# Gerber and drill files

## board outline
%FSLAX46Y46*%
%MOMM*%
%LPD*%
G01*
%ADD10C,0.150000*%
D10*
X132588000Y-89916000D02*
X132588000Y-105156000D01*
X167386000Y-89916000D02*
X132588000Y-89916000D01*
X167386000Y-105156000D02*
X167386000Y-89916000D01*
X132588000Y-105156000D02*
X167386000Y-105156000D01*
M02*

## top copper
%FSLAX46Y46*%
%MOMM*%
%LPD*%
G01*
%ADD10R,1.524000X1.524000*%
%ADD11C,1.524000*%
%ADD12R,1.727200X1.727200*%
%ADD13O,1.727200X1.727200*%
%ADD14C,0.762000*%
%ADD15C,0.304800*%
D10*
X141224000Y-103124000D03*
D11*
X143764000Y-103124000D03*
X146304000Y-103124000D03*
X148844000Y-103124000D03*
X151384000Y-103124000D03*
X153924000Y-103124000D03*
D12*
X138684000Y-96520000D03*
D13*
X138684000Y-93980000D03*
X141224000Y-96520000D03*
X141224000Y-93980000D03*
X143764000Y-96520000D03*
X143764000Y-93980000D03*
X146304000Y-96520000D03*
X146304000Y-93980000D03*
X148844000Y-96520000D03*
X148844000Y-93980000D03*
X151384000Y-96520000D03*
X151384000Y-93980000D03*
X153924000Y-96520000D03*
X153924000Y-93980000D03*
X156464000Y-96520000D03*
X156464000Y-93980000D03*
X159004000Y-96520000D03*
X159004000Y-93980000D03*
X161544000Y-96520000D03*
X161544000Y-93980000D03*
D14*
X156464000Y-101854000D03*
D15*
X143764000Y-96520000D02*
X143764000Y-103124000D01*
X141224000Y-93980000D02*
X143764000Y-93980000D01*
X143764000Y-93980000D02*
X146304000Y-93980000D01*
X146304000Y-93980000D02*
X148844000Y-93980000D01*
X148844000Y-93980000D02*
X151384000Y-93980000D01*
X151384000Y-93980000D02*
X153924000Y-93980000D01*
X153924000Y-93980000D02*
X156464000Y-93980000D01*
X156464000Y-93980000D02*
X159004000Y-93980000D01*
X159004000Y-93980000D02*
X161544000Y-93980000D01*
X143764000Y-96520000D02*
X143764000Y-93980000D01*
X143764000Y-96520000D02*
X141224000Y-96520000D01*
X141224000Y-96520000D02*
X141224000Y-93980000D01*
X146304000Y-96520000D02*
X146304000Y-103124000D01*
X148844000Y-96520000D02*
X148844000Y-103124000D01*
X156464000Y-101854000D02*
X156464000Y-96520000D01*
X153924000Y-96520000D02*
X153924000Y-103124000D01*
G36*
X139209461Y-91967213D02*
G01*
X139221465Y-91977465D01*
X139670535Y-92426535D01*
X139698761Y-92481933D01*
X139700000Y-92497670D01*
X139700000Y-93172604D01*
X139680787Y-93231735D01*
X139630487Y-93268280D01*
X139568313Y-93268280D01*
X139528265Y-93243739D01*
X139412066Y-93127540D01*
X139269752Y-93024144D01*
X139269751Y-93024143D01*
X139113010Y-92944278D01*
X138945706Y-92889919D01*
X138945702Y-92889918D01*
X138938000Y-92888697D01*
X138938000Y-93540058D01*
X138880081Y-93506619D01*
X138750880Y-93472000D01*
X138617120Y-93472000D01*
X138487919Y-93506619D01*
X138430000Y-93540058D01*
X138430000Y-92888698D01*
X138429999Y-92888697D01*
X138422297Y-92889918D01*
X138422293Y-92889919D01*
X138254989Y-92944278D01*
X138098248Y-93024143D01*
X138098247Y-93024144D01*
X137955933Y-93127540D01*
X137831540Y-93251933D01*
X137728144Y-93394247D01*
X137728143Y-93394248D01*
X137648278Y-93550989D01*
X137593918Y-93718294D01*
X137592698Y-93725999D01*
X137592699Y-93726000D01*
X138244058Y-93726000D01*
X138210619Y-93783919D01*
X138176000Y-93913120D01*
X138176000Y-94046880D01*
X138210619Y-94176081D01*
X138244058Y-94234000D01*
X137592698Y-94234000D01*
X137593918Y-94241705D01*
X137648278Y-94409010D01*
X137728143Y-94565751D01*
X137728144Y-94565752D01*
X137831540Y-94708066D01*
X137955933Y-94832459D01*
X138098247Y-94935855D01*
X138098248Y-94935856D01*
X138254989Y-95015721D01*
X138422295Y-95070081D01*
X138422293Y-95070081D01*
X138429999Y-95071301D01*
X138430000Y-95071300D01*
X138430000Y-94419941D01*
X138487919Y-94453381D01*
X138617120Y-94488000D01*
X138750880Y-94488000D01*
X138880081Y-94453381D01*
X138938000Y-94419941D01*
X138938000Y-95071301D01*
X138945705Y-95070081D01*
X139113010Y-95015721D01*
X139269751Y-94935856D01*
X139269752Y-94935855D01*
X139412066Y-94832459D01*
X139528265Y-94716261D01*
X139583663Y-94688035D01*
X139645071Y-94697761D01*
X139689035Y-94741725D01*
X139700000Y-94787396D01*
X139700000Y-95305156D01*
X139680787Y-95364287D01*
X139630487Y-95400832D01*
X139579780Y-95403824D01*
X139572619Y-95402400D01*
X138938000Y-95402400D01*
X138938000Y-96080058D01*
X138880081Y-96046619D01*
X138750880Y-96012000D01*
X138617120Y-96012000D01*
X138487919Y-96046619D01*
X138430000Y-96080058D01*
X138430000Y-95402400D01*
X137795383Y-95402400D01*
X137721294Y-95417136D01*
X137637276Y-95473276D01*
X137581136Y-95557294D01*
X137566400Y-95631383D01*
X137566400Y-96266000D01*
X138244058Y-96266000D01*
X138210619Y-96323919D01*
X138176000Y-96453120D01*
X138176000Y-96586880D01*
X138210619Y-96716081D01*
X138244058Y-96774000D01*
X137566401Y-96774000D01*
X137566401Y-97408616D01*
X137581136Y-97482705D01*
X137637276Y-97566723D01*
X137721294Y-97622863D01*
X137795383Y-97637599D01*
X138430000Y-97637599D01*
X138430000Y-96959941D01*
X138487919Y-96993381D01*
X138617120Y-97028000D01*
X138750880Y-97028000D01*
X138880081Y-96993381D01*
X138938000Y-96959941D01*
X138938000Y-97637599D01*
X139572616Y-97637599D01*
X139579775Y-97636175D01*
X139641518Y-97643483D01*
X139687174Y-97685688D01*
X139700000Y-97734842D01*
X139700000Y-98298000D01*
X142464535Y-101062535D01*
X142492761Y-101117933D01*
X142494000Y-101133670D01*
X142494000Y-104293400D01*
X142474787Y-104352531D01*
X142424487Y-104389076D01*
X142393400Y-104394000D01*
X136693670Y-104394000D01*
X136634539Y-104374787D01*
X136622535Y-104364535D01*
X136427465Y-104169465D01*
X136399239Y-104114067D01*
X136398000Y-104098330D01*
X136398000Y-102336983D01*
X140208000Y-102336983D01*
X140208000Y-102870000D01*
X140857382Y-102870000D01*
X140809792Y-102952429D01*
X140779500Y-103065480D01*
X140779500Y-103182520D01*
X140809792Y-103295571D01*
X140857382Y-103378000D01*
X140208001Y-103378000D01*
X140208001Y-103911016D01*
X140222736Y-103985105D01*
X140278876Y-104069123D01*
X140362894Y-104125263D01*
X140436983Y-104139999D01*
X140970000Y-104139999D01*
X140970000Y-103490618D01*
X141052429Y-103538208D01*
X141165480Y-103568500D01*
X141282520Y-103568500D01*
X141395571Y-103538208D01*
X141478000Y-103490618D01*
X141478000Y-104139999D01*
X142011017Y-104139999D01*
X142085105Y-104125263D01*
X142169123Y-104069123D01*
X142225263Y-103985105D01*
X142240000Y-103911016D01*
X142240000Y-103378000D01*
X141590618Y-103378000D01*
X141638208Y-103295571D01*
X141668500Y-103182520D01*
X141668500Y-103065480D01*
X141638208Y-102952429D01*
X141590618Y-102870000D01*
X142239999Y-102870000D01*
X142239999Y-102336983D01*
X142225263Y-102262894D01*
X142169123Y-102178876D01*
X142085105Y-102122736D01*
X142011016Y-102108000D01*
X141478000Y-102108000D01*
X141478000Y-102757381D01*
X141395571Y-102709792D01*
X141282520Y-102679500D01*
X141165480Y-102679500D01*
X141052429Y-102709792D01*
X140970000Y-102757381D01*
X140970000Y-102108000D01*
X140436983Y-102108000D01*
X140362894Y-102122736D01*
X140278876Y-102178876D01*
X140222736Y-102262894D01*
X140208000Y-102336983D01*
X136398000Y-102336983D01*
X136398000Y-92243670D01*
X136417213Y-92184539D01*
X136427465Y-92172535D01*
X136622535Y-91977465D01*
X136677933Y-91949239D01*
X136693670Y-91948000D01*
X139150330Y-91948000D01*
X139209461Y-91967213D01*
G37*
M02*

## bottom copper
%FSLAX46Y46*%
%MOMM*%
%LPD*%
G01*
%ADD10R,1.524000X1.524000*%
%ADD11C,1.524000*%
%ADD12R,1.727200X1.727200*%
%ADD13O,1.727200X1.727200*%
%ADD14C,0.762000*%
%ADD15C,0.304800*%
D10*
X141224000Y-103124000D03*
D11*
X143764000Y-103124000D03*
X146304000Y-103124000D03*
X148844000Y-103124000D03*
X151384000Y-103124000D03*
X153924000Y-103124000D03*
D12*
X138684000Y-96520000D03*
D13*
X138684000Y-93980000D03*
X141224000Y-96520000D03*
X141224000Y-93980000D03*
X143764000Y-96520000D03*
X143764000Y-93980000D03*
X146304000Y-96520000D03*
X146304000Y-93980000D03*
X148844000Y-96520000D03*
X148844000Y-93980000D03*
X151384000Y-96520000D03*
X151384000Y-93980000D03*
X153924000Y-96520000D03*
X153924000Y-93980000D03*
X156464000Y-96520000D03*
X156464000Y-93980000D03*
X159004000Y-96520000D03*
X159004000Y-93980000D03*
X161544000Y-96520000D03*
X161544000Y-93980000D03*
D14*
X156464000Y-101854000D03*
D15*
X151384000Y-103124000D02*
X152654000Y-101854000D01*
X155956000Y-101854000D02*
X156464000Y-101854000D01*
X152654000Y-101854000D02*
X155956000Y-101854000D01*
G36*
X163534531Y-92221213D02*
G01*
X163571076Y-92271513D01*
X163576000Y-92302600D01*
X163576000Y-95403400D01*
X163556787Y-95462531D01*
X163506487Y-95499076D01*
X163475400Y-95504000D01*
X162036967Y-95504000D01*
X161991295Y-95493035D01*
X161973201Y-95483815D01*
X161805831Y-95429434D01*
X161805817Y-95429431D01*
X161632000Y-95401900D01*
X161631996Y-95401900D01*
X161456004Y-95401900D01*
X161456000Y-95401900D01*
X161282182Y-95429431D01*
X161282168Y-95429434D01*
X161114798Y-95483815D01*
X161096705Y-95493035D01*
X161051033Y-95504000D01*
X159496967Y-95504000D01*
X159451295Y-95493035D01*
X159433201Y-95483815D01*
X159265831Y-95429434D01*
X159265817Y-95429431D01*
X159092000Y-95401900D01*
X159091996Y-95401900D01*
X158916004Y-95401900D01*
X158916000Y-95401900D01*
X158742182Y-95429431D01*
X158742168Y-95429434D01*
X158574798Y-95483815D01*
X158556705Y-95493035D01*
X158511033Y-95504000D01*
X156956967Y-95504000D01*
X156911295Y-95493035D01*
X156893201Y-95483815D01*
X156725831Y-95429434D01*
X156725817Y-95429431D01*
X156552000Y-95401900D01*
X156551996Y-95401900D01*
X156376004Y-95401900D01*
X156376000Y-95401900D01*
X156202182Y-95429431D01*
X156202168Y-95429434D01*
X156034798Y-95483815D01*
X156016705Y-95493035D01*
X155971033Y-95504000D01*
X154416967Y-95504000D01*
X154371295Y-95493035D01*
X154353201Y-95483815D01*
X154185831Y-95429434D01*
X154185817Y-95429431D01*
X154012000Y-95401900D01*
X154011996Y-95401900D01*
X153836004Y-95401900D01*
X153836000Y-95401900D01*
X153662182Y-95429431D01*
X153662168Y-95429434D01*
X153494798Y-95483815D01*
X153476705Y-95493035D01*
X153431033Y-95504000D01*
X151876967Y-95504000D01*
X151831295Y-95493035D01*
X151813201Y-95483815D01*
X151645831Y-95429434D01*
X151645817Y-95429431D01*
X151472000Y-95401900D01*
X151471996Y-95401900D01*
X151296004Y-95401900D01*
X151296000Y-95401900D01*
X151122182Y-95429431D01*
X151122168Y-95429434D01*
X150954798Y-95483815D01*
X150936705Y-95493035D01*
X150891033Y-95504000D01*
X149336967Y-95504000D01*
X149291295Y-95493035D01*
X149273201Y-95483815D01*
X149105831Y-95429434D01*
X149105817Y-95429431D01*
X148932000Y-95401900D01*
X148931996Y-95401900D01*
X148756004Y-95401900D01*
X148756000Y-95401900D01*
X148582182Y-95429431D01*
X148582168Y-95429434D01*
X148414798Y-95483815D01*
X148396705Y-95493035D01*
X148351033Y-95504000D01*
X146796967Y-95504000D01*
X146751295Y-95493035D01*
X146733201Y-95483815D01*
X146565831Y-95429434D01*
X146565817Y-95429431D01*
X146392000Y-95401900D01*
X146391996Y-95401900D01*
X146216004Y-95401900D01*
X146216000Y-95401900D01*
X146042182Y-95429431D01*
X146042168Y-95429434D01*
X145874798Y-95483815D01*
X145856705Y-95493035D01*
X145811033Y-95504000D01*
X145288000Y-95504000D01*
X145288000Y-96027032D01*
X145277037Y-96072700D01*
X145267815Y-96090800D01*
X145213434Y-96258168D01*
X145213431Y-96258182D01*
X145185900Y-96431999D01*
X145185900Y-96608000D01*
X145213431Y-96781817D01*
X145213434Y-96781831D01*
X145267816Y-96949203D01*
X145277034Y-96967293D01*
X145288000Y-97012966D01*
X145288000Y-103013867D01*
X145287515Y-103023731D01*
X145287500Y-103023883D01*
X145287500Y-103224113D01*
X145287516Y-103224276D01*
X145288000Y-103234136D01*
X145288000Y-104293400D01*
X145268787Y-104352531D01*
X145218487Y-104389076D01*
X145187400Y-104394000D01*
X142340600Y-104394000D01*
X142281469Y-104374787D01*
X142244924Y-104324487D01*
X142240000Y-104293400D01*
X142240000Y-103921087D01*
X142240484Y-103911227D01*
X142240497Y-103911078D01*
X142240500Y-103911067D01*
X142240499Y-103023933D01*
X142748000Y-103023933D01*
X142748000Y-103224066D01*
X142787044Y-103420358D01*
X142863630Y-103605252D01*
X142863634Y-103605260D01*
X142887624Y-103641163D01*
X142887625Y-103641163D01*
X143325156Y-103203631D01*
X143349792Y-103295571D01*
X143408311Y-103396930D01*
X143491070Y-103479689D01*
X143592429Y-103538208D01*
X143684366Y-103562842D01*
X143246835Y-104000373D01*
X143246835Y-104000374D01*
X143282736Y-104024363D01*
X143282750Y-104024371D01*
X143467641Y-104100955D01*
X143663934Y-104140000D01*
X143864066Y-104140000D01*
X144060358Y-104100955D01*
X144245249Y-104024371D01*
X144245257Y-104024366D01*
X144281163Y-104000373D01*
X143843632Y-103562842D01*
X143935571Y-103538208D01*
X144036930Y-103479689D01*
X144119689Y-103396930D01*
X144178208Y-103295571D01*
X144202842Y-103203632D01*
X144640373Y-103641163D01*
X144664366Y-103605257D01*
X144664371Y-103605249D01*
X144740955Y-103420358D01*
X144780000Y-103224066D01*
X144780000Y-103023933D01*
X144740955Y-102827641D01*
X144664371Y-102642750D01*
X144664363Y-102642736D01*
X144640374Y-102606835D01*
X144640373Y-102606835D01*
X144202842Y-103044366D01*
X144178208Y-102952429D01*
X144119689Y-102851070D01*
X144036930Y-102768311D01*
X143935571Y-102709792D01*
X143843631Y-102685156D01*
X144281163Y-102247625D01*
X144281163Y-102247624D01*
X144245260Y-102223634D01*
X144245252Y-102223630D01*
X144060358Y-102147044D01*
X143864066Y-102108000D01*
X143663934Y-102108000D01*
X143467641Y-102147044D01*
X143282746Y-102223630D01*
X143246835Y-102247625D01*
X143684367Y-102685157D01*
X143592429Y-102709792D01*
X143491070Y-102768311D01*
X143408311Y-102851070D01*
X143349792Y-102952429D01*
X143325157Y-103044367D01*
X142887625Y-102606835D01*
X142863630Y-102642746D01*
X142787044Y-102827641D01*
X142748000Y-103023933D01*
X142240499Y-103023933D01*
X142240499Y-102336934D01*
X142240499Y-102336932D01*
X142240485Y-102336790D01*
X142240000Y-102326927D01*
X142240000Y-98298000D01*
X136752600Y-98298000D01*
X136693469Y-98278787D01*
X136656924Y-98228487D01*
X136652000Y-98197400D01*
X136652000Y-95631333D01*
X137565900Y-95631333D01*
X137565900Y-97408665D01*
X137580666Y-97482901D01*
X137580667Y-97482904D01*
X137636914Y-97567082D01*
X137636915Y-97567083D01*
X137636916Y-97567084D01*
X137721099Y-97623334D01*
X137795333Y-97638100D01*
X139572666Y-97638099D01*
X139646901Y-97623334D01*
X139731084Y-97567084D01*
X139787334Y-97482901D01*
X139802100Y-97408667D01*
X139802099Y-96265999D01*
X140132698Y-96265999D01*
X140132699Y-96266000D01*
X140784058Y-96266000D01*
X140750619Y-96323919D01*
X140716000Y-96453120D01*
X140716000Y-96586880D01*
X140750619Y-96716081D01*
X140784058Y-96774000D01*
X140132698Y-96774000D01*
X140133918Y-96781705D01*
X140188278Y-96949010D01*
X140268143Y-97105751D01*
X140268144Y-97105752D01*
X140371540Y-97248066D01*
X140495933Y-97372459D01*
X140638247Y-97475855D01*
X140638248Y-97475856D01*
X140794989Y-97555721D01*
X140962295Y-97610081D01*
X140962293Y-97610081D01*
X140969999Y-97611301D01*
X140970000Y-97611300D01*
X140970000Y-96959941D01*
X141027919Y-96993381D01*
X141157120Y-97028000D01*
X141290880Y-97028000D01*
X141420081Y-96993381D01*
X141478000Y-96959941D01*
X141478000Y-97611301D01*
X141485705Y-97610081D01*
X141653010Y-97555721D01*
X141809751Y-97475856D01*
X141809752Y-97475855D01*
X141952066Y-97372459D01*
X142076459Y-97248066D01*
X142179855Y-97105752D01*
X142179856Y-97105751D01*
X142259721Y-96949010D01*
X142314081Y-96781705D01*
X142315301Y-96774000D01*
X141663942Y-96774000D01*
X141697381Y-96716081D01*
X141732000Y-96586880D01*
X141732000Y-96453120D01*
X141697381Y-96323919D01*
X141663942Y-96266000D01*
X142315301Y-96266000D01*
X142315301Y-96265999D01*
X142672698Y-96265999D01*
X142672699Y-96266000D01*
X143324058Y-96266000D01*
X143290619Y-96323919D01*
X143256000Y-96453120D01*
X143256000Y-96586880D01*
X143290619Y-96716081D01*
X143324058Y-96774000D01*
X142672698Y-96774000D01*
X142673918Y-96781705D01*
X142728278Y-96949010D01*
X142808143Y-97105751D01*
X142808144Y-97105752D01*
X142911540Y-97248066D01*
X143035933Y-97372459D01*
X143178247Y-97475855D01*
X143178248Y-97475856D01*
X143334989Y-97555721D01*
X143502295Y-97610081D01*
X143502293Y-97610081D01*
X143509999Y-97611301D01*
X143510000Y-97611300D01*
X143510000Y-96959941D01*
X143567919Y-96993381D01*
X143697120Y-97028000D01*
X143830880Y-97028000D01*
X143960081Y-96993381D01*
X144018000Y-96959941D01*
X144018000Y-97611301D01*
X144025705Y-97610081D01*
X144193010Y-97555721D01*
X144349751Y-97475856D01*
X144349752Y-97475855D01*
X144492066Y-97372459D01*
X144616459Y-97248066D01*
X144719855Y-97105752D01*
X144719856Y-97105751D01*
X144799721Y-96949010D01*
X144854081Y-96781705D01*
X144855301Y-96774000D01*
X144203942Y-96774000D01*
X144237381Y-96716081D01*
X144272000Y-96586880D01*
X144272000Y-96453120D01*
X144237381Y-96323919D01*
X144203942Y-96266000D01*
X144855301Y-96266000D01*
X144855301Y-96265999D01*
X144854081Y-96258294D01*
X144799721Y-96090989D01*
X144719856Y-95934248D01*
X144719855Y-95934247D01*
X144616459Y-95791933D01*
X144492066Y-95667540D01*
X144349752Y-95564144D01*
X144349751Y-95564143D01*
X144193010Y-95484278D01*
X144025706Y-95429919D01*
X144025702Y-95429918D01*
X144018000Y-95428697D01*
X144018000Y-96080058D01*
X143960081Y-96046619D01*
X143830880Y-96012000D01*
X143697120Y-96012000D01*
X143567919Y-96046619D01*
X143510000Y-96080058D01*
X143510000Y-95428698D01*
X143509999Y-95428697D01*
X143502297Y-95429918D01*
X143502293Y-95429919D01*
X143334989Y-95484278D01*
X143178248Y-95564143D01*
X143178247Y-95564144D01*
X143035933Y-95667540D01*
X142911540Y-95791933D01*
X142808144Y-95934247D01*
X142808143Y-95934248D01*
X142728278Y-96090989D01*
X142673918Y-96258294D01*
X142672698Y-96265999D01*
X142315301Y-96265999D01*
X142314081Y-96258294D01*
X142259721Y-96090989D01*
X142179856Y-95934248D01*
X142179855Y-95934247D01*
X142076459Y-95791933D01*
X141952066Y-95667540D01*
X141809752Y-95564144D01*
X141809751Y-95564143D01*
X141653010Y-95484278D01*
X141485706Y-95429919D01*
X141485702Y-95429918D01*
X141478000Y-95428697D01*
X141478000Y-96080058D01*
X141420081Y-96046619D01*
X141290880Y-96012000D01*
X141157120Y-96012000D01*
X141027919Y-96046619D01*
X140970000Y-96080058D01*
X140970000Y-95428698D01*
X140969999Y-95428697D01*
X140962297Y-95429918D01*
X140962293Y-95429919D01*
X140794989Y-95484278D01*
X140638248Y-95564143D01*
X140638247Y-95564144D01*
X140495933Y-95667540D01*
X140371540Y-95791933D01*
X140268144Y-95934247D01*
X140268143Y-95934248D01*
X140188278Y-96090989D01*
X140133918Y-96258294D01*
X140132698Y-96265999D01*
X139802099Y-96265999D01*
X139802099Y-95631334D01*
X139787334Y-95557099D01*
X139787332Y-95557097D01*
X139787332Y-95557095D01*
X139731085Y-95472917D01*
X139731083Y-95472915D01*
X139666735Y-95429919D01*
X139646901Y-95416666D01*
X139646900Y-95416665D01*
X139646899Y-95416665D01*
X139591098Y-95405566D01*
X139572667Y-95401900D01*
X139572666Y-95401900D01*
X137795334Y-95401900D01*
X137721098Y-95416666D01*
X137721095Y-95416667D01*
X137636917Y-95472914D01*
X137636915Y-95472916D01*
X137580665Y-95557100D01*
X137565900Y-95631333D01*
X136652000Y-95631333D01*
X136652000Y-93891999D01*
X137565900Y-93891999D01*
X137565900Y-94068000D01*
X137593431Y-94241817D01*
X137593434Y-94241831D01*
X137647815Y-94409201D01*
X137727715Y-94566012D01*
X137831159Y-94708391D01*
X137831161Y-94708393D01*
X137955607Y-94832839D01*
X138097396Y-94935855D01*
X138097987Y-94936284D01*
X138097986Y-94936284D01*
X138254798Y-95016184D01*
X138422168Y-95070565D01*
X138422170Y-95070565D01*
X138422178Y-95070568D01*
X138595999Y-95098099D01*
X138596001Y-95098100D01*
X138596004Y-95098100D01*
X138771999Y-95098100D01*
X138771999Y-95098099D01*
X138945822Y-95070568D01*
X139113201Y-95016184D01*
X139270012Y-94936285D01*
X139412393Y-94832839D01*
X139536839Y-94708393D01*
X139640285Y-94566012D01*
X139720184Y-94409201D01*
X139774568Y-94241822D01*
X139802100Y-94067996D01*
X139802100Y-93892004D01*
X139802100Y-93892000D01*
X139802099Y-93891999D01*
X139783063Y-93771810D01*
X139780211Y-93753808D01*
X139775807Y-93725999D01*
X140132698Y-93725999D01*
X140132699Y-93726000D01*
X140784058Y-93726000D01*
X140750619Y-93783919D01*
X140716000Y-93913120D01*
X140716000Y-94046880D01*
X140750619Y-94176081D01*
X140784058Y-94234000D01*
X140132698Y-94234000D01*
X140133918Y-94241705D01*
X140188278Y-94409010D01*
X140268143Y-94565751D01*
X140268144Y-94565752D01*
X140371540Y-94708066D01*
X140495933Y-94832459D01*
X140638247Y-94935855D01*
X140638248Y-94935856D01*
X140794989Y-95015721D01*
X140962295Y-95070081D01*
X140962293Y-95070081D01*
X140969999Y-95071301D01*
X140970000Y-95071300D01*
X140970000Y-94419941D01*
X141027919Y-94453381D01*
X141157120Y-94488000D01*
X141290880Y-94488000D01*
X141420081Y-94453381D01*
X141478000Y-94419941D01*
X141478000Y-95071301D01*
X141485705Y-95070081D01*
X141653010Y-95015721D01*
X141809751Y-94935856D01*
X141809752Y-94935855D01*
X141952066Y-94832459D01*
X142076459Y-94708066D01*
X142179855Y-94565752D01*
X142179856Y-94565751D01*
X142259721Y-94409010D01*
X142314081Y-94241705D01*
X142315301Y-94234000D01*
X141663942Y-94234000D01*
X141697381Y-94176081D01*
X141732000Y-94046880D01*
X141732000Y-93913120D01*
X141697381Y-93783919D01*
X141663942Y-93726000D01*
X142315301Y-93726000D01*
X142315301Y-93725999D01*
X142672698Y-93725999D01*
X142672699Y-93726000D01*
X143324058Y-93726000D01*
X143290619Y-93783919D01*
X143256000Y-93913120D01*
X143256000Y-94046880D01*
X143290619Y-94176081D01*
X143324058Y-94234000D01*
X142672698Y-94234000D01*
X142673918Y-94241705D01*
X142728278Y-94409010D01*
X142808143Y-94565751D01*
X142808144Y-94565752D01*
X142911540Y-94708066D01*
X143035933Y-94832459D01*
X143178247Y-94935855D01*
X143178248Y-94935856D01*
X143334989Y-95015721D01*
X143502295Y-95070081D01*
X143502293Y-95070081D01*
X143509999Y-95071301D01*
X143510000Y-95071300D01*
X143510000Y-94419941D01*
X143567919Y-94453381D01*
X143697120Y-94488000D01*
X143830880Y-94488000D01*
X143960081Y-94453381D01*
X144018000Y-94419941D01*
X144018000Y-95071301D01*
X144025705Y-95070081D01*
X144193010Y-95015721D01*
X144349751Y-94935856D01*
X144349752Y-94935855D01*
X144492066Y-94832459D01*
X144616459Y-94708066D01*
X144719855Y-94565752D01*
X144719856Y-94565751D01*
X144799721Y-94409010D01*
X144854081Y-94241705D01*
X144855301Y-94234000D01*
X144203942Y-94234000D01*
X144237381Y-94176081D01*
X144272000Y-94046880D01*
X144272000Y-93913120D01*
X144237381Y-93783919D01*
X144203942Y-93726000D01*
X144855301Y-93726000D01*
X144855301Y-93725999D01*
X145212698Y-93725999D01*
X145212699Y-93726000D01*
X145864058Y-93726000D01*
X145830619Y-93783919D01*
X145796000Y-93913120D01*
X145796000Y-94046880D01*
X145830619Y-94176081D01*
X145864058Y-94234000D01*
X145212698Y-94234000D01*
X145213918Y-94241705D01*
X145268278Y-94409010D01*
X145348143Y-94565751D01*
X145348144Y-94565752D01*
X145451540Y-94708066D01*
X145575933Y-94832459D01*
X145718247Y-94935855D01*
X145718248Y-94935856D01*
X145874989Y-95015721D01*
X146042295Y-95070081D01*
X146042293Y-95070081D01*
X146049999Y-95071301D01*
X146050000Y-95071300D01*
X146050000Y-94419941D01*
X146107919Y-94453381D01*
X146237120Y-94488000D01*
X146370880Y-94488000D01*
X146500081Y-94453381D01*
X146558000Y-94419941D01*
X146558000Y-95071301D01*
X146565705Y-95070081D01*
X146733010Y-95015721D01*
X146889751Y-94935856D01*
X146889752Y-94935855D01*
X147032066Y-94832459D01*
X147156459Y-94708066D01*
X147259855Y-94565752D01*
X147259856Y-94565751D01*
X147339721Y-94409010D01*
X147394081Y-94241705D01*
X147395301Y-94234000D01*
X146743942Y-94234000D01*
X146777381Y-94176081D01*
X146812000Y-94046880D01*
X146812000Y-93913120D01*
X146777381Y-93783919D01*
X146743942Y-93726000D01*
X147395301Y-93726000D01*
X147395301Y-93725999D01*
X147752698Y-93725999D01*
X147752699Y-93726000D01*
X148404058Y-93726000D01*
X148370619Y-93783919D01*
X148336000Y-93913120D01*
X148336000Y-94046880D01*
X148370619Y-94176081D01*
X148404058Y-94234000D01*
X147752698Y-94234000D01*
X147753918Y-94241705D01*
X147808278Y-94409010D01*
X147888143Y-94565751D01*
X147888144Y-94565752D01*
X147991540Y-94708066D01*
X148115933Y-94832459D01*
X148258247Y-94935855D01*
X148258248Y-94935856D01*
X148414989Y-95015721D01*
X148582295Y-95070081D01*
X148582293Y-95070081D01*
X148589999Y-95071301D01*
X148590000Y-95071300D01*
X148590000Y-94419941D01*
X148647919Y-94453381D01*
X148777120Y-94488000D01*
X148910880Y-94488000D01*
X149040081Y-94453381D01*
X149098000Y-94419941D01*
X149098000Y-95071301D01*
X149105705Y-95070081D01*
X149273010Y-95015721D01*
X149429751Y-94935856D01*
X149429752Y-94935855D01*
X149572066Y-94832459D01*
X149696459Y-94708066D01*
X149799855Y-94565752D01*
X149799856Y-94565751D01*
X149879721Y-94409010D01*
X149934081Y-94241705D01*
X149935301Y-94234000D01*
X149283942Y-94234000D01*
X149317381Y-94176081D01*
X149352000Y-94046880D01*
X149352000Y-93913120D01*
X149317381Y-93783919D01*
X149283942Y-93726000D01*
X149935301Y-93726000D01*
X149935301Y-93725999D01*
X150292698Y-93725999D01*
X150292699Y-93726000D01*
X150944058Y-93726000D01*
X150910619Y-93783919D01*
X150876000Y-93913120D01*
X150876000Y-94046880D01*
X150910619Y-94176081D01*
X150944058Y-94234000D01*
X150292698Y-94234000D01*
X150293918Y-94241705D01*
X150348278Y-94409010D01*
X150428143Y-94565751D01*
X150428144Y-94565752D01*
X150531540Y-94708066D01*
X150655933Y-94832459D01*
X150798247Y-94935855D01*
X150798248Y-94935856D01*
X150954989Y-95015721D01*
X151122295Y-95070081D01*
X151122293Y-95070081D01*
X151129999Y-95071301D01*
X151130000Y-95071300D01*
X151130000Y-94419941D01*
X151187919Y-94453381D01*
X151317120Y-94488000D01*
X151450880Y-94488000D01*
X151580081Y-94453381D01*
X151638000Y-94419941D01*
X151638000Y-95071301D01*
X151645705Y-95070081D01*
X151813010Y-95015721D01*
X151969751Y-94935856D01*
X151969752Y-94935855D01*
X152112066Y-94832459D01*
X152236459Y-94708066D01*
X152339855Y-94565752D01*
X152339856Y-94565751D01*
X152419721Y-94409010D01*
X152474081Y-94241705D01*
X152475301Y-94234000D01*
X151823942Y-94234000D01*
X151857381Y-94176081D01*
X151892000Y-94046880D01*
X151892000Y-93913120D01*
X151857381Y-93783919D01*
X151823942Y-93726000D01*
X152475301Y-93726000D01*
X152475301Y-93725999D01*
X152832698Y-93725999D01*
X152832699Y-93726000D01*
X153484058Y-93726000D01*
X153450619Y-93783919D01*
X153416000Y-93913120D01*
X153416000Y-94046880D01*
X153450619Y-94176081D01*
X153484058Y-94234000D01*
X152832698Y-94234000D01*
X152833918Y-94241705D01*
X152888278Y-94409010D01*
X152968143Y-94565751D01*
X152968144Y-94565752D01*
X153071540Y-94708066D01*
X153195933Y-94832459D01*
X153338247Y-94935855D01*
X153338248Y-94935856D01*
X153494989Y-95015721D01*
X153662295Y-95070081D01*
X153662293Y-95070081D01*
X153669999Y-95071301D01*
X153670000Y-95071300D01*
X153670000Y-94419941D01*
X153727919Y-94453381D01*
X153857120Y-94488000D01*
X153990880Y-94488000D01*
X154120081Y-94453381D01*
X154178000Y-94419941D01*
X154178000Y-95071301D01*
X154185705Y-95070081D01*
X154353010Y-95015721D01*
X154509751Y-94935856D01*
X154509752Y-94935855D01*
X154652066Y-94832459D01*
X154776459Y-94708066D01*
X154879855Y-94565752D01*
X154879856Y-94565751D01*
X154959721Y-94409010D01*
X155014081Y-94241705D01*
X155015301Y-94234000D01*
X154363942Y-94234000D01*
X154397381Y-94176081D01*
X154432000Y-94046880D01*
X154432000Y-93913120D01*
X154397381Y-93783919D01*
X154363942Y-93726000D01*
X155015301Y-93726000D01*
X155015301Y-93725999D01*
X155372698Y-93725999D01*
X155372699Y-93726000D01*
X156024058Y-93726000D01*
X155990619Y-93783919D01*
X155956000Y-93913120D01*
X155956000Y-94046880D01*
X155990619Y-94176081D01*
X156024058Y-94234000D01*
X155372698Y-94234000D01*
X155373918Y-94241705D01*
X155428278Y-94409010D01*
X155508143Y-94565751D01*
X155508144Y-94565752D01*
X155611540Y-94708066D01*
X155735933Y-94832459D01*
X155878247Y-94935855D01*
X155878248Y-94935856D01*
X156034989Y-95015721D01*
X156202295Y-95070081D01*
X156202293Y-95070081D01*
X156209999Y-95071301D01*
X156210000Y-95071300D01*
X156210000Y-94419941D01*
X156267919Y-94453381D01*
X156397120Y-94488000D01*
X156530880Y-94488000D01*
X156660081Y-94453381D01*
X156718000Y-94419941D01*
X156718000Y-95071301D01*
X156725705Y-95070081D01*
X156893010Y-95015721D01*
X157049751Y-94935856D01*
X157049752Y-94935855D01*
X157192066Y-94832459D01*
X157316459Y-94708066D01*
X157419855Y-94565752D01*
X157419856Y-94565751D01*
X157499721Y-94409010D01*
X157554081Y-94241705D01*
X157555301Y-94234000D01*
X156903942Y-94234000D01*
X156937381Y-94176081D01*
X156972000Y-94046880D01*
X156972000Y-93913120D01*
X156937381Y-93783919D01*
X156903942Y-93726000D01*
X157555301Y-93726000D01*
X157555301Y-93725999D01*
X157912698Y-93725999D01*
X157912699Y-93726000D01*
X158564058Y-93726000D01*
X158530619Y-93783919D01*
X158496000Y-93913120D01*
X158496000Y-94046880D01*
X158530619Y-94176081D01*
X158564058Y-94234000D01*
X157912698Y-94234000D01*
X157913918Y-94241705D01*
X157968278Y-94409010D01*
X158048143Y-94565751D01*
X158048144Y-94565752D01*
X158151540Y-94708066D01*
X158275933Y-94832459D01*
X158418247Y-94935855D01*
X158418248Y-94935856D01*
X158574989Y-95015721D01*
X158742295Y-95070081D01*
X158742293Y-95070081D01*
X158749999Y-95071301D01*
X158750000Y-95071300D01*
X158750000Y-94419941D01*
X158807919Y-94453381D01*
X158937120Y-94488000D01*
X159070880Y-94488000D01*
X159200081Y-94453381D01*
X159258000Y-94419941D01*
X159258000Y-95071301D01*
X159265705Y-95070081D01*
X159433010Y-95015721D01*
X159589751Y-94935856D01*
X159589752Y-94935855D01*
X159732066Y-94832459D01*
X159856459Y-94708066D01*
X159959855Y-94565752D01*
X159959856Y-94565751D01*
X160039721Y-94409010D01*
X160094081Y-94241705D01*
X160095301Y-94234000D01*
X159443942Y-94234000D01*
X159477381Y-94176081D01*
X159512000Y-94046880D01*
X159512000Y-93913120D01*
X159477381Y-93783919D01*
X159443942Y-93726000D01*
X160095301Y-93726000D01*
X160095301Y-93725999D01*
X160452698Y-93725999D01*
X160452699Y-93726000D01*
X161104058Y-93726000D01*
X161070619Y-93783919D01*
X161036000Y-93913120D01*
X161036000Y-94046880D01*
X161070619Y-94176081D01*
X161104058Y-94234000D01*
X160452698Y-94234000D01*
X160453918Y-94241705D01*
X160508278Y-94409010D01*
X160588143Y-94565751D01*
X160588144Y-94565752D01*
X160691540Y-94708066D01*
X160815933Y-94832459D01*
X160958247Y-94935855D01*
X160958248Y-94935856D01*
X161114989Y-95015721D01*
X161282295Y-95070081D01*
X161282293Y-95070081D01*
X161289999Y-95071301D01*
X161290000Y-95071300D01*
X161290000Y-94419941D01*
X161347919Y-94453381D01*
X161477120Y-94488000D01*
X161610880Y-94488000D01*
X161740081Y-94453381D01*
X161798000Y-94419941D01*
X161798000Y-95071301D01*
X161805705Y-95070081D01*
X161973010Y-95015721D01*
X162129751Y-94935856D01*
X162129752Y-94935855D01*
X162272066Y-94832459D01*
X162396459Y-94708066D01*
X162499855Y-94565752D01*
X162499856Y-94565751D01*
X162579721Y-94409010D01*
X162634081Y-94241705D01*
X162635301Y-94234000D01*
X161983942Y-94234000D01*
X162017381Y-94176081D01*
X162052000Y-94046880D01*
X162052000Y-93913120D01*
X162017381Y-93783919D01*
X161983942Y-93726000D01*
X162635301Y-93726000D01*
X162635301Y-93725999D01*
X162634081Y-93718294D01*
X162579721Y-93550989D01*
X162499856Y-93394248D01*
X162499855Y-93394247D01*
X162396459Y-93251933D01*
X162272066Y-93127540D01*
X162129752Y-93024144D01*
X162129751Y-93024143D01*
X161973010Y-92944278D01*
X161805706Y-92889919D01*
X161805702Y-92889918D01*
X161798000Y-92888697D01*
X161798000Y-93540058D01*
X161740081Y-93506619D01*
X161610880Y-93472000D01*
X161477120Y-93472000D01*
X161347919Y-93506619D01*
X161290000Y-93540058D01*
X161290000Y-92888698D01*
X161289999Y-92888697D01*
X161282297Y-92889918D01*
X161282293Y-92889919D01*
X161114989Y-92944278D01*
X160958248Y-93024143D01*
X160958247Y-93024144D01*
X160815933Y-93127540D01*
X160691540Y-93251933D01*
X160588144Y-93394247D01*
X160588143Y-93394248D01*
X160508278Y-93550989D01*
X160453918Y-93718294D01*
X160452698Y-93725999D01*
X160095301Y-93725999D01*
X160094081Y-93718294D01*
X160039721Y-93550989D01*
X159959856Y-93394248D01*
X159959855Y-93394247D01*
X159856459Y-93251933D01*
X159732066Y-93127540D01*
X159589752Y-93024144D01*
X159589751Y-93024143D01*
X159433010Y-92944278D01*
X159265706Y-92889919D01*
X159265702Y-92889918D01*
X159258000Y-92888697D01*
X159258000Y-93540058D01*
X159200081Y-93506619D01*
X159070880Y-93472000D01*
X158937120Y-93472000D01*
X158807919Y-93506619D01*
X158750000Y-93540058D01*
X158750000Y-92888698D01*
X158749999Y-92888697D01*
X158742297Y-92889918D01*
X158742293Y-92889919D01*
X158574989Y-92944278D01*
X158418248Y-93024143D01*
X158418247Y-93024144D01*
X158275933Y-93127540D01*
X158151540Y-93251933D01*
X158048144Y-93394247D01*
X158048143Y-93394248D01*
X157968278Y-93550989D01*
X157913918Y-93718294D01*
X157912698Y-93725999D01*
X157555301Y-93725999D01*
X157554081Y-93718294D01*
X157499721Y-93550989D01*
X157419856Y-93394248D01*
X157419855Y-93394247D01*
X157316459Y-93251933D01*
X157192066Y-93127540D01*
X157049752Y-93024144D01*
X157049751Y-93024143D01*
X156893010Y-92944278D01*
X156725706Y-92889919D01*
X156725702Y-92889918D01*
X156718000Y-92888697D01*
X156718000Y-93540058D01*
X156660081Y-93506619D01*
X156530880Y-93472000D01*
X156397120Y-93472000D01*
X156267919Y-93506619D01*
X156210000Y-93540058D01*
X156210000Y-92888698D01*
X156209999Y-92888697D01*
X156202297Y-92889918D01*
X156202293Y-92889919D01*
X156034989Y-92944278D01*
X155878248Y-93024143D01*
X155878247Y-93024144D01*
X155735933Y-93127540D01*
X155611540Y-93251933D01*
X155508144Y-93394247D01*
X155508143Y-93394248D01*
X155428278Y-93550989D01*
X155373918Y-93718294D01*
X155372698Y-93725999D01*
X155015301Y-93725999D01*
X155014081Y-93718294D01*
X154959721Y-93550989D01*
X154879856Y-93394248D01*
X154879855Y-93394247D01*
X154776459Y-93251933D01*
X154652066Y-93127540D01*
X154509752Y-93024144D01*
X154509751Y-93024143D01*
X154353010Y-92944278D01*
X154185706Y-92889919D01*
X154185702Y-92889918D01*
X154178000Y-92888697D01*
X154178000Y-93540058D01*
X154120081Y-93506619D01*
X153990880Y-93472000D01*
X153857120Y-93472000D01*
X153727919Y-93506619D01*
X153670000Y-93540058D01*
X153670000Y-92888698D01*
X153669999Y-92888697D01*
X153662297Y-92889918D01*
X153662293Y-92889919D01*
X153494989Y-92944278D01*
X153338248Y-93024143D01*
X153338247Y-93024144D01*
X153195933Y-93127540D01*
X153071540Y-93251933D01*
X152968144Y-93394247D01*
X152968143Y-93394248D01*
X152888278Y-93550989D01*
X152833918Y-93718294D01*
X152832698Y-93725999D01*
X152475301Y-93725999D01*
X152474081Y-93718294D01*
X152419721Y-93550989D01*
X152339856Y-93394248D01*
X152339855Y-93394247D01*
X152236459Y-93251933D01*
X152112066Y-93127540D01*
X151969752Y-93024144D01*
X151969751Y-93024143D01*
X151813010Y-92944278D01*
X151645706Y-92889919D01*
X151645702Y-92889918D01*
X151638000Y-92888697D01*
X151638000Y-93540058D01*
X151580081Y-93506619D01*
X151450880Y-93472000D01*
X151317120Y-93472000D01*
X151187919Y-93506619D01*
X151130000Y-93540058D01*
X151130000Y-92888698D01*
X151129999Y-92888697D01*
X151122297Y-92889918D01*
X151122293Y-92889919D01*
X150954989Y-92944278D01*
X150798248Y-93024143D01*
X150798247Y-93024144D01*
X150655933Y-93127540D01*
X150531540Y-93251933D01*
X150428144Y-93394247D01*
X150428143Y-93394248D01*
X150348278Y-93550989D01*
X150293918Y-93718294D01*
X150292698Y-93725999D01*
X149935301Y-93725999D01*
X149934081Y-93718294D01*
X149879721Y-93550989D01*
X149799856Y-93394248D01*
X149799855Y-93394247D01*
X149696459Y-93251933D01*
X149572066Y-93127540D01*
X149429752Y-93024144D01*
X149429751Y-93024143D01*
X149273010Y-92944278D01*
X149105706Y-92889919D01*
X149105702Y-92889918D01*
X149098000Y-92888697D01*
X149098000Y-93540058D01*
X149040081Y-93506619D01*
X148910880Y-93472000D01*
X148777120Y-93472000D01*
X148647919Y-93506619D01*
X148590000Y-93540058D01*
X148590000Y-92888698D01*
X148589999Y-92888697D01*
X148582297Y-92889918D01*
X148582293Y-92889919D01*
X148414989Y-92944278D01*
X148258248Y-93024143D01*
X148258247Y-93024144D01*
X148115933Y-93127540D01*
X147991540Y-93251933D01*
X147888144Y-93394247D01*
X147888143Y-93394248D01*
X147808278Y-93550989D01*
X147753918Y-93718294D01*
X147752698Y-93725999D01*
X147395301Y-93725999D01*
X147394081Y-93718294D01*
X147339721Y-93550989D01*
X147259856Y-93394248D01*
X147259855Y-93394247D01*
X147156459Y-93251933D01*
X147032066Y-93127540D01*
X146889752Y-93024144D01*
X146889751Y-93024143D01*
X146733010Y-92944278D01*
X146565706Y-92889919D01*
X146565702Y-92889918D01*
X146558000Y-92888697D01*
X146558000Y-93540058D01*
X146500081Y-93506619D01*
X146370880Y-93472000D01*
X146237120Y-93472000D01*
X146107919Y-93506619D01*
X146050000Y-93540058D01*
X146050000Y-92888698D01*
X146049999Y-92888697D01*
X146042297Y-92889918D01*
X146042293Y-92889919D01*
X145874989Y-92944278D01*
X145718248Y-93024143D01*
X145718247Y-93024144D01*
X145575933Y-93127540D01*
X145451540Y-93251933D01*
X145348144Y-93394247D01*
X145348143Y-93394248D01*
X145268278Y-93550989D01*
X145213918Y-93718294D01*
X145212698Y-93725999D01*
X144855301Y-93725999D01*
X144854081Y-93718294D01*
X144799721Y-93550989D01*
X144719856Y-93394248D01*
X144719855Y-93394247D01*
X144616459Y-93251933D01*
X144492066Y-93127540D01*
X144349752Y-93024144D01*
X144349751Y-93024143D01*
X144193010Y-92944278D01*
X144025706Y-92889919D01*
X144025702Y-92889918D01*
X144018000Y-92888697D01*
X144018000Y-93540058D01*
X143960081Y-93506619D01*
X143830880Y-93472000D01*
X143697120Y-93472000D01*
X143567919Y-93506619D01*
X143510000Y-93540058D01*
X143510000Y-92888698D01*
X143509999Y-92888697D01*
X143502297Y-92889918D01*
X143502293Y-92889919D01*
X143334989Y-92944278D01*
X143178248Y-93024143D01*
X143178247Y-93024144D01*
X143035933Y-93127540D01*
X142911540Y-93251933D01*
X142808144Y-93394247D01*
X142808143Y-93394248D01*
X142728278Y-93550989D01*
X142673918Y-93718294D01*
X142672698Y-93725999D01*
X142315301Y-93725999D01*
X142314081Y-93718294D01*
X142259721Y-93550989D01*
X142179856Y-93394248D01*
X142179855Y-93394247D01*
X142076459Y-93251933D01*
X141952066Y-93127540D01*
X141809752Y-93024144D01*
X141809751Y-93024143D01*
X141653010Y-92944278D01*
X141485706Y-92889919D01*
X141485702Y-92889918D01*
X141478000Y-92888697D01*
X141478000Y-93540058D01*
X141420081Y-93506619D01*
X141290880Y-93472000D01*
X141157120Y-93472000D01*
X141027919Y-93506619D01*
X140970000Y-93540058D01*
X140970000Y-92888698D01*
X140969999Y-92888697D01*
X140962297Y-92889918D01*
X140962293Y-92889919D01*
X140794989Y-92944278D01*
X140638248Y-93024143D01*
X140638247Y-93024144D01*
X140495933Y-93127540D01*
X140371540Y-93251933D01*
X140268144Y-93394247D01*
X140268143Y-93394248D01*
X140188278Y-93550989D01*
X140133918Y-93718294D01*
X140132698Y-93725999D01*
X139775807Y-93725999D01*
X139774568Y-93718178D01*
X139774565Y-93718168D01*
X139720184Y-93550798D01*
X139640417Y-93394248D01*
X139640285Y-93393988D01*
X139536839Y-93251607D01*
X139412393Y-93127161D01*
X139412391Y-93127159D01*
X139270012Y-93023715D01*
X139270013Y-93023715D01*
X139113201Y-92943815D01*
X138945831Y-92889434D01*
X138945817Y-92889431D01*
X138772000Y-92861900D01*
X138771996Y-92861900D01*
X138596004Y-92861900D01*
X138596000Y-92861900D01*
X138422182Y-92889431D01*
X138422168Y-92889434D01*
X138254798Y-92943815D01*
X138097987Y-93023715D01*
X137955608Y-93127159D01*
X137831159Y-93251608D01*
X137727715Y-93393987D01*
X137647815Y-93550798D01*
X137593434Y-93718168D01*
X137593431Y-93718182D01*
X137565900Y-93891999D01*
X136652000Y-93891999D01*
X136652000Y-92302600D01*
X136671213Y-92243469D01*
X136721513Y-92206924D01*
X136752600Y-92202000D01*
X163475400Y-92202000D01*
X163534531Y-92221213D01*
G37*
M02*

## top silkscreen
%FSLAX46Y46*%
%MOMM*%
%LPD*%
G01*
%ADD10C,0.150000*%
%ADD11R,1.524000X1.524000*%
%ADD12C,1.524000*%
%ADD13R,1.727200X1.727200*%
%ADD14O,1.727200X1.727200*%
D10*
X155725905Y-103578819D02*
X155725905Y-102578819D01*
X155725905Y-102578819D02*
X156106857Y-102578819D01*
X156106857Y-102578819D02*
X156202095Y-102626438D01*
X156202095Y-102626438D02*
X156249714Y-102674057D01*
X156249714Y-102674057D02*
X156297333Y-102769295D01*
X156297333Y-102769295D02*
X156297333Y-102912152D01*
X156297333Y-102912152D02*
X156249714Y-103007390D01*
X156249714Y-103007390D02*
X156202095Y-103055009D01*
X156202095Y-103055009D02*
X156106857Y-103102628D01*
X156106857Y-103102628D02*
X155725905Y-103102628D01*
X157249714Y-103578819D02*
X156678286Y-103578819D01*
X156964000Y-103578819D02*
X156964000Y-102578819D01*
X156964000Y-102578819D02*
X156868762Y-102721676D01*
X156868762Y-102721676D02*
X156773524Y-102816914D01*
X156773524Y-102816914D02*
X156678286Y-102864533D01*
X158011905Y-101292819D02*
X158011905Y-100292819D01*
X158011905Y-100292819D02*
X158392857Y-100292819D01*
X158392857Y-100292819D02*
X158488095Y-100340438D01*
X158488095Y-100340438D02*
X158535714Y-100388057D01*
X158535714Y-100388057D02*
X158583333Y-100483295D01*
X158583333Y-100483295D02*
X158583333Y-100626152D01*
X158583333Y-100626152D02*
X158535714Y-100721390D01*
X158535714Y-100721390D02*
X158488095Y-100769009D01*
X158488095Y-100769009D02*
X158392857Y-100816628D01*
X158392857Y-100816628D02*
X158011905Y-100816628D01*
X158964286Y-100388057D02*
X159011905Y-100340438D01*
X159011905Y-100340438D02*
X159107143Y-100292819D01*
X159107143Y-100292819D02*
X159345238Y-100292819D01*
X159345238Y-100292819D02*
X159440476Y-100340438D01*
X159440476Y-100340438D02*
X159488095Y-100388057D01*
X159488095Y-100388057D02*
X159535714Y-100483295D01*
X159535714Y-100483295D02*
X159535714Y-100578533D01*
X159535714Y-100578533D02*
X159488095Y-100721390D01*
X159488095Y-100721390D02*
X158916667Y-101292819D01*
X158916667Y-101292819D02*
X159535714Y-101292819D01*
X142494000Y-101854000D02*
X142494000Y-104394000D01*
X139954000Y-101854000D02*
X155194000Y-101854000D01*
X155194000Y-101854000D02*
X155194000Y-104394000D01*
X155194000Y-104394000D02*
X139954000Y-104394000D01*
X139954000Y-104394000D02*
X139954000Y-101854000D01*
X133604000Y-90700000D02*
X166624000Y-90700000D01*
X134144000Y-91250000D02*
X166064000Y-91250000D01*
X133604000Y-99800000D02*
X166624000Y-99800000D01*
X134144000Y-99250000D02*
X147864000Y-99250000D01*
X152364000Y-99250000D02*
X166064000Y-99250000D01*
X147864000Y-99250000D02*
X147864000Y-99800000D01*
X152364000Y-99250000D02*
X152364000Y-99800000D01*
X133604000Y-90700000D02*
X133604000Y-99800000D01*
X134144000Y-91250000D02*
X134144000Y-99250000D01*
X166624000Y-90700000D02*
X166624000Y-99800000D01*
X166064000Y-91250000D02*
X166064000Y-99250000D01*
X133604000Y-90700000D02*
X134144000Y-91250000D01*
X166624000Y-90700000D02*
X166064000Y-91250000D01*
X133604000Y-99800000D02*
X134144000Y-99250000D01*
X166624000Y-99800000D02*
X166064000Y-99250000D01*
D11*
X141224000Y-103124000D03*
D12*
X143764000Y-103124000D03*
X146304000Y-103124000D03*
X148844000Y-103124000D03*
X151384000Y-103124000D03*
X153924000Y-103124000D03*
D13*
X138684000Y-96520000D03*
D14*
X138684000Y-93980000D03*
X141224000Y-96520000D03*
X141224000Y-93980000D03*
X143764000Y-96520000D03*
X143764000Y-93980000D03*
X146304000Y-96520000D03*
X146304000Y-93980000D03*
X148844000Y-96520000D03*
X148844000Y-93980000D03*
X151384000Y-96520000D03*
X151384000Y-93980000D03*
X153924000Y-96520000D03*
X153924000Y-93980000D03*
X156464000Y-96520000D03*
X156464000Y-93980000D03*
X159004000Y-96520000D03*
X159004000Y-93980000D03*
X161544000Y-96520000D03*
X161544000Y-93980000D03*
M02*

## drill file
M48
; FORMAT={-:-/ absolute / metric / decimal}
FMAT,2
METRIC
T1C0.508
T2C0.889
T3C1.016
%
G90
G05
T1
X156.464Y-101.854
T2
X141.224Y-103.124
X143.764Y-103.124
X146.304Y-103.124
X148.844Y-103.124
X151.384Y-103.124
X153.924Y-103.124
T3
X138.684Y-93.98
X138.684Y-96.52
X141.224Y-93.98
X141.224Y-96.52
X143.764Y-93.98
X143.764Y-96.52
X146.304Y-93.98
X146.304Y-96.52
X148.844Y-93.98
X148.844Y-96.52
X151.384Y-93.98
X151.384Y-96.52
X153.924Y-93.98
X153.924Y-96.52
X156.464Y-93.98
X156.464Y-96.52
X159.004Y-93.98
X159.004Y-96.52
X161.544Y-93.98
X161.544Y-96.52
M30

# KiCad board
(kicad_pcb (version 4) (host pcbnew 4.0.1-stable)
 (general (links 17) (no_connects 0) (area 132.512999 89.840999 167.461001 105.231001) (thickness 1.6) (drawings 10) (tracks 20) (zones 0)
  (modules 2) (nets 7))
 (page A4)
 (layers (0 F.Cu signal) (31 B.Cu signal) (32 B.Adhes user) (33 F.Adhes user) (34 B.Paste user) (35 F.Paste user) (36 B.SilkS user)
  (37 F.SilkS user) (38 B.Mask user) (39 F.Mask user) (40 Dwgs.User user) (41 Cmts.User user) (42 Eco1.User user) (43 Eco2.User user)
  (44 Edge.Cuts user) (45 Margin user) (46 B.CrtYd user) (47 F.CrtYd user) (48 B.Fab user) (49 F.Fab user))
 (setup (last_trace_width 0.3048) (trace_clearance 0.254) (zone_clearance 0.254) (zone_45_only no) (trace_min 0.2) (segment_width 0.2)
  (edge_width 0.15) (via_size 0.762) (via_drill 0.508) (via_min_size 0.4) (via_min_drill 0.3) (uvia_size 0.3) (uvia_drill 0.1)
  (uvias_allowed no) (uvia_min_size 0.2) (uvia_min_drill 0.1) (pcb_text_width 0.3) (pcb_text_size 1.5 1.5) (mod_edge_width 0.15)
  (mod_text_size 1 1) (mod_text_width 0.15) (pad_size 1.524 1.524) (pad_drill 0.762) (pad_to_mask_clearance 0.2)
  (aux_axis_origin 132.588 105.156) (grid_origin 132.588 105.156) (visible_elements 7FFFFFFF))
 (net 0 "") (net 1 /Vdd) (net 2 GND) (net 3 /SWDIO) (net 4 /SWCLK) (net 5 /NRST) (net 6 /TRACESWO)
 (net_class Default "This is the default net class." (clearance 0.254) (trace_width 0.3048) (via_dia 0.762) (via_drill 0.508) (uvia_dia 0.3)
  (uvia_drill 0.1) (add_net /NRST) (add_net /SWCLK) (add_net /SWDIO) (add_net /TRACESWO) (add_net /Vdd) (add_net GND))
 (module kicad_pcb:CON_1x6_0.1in (layer F.Cu) (at 147.574 103.124)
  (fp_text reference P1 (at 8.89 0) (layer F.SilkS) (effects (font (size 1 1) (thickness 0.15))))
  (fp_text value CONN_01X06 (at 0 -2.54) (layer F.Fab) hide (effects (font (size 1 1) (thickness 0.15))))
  (fp_line (start -5.08 -1.27) (end -5.08 1.27) (layer F.SilkS) (width 0.15))
  (fp_line (start -7.62 -1.27) (end 7.62 -1.27) (layer F.SilkS) (width 0.15))
  (fp_line (start 7.62 -1.27) (end 7.62 1.27) (layer F.SilkS) (width 0.15))
  (fp_line (start 7.62 1.27) (end -7.62 1.27) (layer F.SilkS) (width 0.15))
  (fp_line (start -7.62 1.27) (end -7.62 -1.27) (layer F.SilkS) (width 0.15))
  (pad 1 thru_hole rect (at -6.35 0) (size 1.524 1.524) (drill 0.889) (layers *.Cu *.Mask F.SilkS) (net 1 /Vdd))
  (pad 2 thru_hole circle (at -3.81 0) (size 1.524 1.524) (drill 0.889) (layers *.Cu *.Mask F.SilkS) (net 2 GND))
  (pad 3 thru_hole circle (at -1.27 0) (size 1.524 1.524) (drill 0.889) (layers *.Cu *.Mask F.SilkS) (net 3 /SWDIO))
  (pad 4 thru_hole circle (at 1.27 0) (size 1.524 1.524) (drill 0.889) (layers *.Cu *.Mask F.SilkS) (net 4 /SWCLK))
  (pad 5 thru_hole circle (at 3.81 0) (size 1.524 1.524) (drill 0.889) (layers *.Cu *.Mask F.SilkS) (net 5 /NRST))
  (pad 6 thru_hole circle (at 6.35 0) (size 1.524 1.524) (drill 0.889) (layers *.Cu *.Mask F.SilkS) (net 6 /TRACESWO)))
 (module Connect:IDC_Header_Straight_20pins (layer F.Cu) (at 138.684 96.52)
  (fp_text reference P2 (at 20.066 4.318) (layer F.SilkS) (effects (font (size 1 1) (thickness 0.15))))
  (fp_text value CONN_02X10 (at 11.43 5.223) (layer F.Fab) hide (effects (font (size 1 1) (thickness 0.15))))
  (fp_line (start -5.08 -5.82) (end 27.94 -5.82) (layer F.SilkS) (width 0.15))
  (fp_line (start -4.54 -5.27) (end 27.38 -5.27) (layer F.SilkS) (width 0.15))
  (fp_line (start -5.08 3.28) (end 27.94 3.28) (layer F.SilkS) (width 0.15))
  (fp_line (start -4.54 2.73) (end 9.18 2.73) (layer F.SilkS) (width 0.15))
  (fp_line (start 13.68 2.73) (end 27.38 2.73) (layer F.SilkS) (width 0.15))
  (fp_line (start 9.18 2.73) (end 9.18 3.28) (layer F.SilkS) (width 0.15))
  (fp_line (start 13.68 2.73) (end 13.68 3.28) (layer F.SilkS) (width 0.15))
  (fp_line (start -5.08 -5.82) (end -5.08 3.28) (layer F.SilkS) (width 0.15))
  (fp_line (start -4.54 -5.27) (end -4.54 2.73) (layer F.SilkS) (width 0.15))
  (fp_line (start 27.94 -5.82) (end 27.94 3.28) (layer F.SilkS) (width 0.15))
  (fp_line (start 27.38 -5.27) (end 27.38 2.73) (layer F.SilkS) (width 0.15))
  (fp_line (start -5.08 -5.82) (end -4.54 -5.27) (layer F.SilkS) (width 0.15))
  (fp_line (start 27.94 -5.82) (end 27.38 -5.27) (layer F.SilkS) (width 0.15))
  (fp_line (start -5.08 3.28) (end -4.54 2.73) (layer F.SilkS) (width 0.15))
  (fp_line (start 27.94 3.28) (end 27.38 2.73) (layer F.SilkS) (width 0.15))
  (pad 1 thru_hole rect (at 0 0) (size 1.7272 1.7272) (drill 1.016) (layers *.Cu *.Mask F.SilkS) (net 1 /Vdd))
  (pad 2 thru_hole oval (at 0 -2.54) (size 1.7272 1.7272) (drill 1.016) (layers *.Cu *.Mask F.SilkS) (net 1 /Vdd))
  (pad 3 thru_hole oval (at 2.54 0) (size 1.7272 1.7272) (drill 1.016) (layers *.Cu *.Mask F.SilkS) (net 2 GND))
  (pad 4 thru_hole oval (at 2.54 -2.54) (size 1.7272 1.7272) (drill 1.016) (layers *.Cu *.Mask F.SilkS) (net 2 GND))
  (pad 5 thru_hole oval (at 5.08 0) (size 1.7272 1.7272) (drill 1.016) (layers *.Cu *.Mask F.SilkS) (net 2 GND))
  (pad 6 thru_hole oval (at 5.08 -2.54) (size 1.7272 1.7272) (drill 1.016) (layers *.Cu *.Mask F.SilkS) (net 2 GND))
  (pad 7 thru_hole oval (at 7.62 0) (size 1.7272 1.7272) (drill 1.016) (layers *.Cu *.Mask F.SilkS) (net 3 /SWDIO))
  (pad 8 thru_hole oval (at 7.62 -2.54) (size 1.7272 1.7272) (drill 1.016) (layers *.Cu *.Mask F.SilkS) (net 2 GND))
  (pad 9 thru_hole oval (at 10.16 0) (size 1.7272 1.7272) (drill 1.016) (layers *.Cu *.Mask F.SilkS) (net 4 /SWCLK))
  (pad 10 thru_hole oval (at 10.16 -2.54) (size 1.7272 1.7272) (drill 1.016) (layers *.Cu *.Mask F.SilkS) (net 2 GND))
  (pad 11 thru_hole oval (at 12.7 0) (size 1.7272 1.7272) (drill 1.016) (layers *.Cu *.Mask F.SilkS))
  (pad 12 thru_hole oval (at 12.7 -2.54) (size 1.7272 1.7272) (drill 1.016) (layers *.Cu *.Mask F.SilkS) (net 2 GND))
  (pad 13 thru_hole oval (at 15.24 0) (size 1.7272 1.7272) (drill 1.016) (layers *.Cu *.Mask F.SilkS) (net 6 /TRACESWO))
  (pad 14 thru_hole oval (at 15.24 -2.54) (size 1.7272 1.7272) (drill 1.016) (layers *.Cu *.Mask F.SilkS) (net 2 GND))
  (pad 15 thru_hole oval (at 17.78 0) (size 1.7272 1.7272) (drill 1.016) (layers *.Cu *.Mask F.SilkS) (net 5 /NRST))
  (pad 16 thru_hole oval (at 17.78 -2.54) (size 1.7272 1.7272) (drill 1.016) (layers *.Cu *.Mask F.SilkS) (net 2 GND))
  (pad 17 thru_hole oval (at 20.32 0) (size 1.7272 1.7272) (drill 1.016) (layers *.Cu *.Mask F.SilkS))
  (pad 18 thru_hole oval (at 20.32 -2.54) (size 1.7272 1.7272) (drill 1.016) (layers *.Cu *.Mask F.SilkS) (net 2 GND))
  (pad 19 thru_hole oval (at 22.86 0) (size 1.7272 1.7272) (drill 1.016) (layers *.Cu *.Mask F.SilkS))
  (pad 20 thru_hole oval (at 22.86 -2.54) (size 1.7272 1.7272) (drill 1.016) (layers *.Cu *.Mask F.SilkS) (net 2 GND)))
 (gr_line (start 132.588 89.916) (end 132.588 105.156) (angle 90) (layer Edge.Cuts) (width 0.15))
 (gr_line (start 167.386 89.916) (end 132.588 89.916) (angle 90) (layer Edge.Cuts) (width 0.15))
 (gr_line (start 167.386 105.156) (end 167.386 89.916) (angle 90) (layer Edge.Cuts) (width 0.15))
 (gr_line (start 132.588 105.156) (end 167.386 105.156) (angle 90) (layer Edge.Cuts) (width 0.15))
 (segment (start 143.764 96.52) (end 143.764 103.124) (width 0.3048) (layer F.Cu) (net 2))
 (segment (start 141.224 93.98) (end 143.764 93.98) (width 0.3048) (layer F.Cu) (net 2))
 (segment (start 143.764 93.98) (end 146.304 93.98) (width 0.3048) (layer F.Cu) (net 2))
 (segment (start 146.304 93.98) (end 148.844 93.98) (width 0.3048) (layer F.Cu) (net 2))
 (segment (start 148.844 93.98) (end 151.384 93.98) (width 0.3048) (layer F.Cu) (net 2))
 (segment (start 151.384 93.98) (end 153.924 93.98) (width 0.3048) (layer F.Cu) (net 2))
 (segment (start 153.924 93.98) (end 156.464 93.98) (width 0.3048) (layer F.Cu) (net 2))
 (segment (start 156.464 93.98) (end 159.004 93.98) (width 0.3048) (layer F.Cu) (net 2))
 (segment (start 159.004 93.98) (end 161.544 93.98) (width 0.3048) (layer F.Cu) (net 2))
 (segment (start 143.764 96.52) (end 143.764 93.98) (width 0.3048) (layer F.Cu) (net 2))
 (segment (start 143.764 96.52) (end 141.224 96.52) (width 0.3048) (layer F.Cu) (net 2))
 (segment (start 141.224 96.52) (end 141.224 93.98) (width 0.3048) (layer F.Cu) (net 2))
 (segment (start 146.304 96.52) (end 146.304 103.124) (width 0.3048) (layer F.Cu) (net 3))
 (segment (start 148.844 96.52) (end 148.844 103.124) (width 0.3048) (layer F.Cu) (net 4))
 (segment (start 151.384 103.124) (end 152.654 101.854) (width 0.3048) (layer B.Cu) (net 5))
 (segment (start 156.464 101.854) (end 156.464 96.52) (width 0.3048) (layer F.Cu) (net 5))
 (via (at 156.464 101.854) (size 0.762) (drill 0.508) (layers F.Cu B.Cu) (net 5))
 (segment (start 155.956 101.854) (end 156.464 101.854) (width 0.3048) (layer B.Cu) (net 5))
 (segment (start 152.654 101.854) (end 155.956 101.854) (width 0.3048) (layer B.Cu) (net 5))
 (segment (start 153.924 96.52) (end 153.924 103.124) (width 0.3048) (layer F.Cu) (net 6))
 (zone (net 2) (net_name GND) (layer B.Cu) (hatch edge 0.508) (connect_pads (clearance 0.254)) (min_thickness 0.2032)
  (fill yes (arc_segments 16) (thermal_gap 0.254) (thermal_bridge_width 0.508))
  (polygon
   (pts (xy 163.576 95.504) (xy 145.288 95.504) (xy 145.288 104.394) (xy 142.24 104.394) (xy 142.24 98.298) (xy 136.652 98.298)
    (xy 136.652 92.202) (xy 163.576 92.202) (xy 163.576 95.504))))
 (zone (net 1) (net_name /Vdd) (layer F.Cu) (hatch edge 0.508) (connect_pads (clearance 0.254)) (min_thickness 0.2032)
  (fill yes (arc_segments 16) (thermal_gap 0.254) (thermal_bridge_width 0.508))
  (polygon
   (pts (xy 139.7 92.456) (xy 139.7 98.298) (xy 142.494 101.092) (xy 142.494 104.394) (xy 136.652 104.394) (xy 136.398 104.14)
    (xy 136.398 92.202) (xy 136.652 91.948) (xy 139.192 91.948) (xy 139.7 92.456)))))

